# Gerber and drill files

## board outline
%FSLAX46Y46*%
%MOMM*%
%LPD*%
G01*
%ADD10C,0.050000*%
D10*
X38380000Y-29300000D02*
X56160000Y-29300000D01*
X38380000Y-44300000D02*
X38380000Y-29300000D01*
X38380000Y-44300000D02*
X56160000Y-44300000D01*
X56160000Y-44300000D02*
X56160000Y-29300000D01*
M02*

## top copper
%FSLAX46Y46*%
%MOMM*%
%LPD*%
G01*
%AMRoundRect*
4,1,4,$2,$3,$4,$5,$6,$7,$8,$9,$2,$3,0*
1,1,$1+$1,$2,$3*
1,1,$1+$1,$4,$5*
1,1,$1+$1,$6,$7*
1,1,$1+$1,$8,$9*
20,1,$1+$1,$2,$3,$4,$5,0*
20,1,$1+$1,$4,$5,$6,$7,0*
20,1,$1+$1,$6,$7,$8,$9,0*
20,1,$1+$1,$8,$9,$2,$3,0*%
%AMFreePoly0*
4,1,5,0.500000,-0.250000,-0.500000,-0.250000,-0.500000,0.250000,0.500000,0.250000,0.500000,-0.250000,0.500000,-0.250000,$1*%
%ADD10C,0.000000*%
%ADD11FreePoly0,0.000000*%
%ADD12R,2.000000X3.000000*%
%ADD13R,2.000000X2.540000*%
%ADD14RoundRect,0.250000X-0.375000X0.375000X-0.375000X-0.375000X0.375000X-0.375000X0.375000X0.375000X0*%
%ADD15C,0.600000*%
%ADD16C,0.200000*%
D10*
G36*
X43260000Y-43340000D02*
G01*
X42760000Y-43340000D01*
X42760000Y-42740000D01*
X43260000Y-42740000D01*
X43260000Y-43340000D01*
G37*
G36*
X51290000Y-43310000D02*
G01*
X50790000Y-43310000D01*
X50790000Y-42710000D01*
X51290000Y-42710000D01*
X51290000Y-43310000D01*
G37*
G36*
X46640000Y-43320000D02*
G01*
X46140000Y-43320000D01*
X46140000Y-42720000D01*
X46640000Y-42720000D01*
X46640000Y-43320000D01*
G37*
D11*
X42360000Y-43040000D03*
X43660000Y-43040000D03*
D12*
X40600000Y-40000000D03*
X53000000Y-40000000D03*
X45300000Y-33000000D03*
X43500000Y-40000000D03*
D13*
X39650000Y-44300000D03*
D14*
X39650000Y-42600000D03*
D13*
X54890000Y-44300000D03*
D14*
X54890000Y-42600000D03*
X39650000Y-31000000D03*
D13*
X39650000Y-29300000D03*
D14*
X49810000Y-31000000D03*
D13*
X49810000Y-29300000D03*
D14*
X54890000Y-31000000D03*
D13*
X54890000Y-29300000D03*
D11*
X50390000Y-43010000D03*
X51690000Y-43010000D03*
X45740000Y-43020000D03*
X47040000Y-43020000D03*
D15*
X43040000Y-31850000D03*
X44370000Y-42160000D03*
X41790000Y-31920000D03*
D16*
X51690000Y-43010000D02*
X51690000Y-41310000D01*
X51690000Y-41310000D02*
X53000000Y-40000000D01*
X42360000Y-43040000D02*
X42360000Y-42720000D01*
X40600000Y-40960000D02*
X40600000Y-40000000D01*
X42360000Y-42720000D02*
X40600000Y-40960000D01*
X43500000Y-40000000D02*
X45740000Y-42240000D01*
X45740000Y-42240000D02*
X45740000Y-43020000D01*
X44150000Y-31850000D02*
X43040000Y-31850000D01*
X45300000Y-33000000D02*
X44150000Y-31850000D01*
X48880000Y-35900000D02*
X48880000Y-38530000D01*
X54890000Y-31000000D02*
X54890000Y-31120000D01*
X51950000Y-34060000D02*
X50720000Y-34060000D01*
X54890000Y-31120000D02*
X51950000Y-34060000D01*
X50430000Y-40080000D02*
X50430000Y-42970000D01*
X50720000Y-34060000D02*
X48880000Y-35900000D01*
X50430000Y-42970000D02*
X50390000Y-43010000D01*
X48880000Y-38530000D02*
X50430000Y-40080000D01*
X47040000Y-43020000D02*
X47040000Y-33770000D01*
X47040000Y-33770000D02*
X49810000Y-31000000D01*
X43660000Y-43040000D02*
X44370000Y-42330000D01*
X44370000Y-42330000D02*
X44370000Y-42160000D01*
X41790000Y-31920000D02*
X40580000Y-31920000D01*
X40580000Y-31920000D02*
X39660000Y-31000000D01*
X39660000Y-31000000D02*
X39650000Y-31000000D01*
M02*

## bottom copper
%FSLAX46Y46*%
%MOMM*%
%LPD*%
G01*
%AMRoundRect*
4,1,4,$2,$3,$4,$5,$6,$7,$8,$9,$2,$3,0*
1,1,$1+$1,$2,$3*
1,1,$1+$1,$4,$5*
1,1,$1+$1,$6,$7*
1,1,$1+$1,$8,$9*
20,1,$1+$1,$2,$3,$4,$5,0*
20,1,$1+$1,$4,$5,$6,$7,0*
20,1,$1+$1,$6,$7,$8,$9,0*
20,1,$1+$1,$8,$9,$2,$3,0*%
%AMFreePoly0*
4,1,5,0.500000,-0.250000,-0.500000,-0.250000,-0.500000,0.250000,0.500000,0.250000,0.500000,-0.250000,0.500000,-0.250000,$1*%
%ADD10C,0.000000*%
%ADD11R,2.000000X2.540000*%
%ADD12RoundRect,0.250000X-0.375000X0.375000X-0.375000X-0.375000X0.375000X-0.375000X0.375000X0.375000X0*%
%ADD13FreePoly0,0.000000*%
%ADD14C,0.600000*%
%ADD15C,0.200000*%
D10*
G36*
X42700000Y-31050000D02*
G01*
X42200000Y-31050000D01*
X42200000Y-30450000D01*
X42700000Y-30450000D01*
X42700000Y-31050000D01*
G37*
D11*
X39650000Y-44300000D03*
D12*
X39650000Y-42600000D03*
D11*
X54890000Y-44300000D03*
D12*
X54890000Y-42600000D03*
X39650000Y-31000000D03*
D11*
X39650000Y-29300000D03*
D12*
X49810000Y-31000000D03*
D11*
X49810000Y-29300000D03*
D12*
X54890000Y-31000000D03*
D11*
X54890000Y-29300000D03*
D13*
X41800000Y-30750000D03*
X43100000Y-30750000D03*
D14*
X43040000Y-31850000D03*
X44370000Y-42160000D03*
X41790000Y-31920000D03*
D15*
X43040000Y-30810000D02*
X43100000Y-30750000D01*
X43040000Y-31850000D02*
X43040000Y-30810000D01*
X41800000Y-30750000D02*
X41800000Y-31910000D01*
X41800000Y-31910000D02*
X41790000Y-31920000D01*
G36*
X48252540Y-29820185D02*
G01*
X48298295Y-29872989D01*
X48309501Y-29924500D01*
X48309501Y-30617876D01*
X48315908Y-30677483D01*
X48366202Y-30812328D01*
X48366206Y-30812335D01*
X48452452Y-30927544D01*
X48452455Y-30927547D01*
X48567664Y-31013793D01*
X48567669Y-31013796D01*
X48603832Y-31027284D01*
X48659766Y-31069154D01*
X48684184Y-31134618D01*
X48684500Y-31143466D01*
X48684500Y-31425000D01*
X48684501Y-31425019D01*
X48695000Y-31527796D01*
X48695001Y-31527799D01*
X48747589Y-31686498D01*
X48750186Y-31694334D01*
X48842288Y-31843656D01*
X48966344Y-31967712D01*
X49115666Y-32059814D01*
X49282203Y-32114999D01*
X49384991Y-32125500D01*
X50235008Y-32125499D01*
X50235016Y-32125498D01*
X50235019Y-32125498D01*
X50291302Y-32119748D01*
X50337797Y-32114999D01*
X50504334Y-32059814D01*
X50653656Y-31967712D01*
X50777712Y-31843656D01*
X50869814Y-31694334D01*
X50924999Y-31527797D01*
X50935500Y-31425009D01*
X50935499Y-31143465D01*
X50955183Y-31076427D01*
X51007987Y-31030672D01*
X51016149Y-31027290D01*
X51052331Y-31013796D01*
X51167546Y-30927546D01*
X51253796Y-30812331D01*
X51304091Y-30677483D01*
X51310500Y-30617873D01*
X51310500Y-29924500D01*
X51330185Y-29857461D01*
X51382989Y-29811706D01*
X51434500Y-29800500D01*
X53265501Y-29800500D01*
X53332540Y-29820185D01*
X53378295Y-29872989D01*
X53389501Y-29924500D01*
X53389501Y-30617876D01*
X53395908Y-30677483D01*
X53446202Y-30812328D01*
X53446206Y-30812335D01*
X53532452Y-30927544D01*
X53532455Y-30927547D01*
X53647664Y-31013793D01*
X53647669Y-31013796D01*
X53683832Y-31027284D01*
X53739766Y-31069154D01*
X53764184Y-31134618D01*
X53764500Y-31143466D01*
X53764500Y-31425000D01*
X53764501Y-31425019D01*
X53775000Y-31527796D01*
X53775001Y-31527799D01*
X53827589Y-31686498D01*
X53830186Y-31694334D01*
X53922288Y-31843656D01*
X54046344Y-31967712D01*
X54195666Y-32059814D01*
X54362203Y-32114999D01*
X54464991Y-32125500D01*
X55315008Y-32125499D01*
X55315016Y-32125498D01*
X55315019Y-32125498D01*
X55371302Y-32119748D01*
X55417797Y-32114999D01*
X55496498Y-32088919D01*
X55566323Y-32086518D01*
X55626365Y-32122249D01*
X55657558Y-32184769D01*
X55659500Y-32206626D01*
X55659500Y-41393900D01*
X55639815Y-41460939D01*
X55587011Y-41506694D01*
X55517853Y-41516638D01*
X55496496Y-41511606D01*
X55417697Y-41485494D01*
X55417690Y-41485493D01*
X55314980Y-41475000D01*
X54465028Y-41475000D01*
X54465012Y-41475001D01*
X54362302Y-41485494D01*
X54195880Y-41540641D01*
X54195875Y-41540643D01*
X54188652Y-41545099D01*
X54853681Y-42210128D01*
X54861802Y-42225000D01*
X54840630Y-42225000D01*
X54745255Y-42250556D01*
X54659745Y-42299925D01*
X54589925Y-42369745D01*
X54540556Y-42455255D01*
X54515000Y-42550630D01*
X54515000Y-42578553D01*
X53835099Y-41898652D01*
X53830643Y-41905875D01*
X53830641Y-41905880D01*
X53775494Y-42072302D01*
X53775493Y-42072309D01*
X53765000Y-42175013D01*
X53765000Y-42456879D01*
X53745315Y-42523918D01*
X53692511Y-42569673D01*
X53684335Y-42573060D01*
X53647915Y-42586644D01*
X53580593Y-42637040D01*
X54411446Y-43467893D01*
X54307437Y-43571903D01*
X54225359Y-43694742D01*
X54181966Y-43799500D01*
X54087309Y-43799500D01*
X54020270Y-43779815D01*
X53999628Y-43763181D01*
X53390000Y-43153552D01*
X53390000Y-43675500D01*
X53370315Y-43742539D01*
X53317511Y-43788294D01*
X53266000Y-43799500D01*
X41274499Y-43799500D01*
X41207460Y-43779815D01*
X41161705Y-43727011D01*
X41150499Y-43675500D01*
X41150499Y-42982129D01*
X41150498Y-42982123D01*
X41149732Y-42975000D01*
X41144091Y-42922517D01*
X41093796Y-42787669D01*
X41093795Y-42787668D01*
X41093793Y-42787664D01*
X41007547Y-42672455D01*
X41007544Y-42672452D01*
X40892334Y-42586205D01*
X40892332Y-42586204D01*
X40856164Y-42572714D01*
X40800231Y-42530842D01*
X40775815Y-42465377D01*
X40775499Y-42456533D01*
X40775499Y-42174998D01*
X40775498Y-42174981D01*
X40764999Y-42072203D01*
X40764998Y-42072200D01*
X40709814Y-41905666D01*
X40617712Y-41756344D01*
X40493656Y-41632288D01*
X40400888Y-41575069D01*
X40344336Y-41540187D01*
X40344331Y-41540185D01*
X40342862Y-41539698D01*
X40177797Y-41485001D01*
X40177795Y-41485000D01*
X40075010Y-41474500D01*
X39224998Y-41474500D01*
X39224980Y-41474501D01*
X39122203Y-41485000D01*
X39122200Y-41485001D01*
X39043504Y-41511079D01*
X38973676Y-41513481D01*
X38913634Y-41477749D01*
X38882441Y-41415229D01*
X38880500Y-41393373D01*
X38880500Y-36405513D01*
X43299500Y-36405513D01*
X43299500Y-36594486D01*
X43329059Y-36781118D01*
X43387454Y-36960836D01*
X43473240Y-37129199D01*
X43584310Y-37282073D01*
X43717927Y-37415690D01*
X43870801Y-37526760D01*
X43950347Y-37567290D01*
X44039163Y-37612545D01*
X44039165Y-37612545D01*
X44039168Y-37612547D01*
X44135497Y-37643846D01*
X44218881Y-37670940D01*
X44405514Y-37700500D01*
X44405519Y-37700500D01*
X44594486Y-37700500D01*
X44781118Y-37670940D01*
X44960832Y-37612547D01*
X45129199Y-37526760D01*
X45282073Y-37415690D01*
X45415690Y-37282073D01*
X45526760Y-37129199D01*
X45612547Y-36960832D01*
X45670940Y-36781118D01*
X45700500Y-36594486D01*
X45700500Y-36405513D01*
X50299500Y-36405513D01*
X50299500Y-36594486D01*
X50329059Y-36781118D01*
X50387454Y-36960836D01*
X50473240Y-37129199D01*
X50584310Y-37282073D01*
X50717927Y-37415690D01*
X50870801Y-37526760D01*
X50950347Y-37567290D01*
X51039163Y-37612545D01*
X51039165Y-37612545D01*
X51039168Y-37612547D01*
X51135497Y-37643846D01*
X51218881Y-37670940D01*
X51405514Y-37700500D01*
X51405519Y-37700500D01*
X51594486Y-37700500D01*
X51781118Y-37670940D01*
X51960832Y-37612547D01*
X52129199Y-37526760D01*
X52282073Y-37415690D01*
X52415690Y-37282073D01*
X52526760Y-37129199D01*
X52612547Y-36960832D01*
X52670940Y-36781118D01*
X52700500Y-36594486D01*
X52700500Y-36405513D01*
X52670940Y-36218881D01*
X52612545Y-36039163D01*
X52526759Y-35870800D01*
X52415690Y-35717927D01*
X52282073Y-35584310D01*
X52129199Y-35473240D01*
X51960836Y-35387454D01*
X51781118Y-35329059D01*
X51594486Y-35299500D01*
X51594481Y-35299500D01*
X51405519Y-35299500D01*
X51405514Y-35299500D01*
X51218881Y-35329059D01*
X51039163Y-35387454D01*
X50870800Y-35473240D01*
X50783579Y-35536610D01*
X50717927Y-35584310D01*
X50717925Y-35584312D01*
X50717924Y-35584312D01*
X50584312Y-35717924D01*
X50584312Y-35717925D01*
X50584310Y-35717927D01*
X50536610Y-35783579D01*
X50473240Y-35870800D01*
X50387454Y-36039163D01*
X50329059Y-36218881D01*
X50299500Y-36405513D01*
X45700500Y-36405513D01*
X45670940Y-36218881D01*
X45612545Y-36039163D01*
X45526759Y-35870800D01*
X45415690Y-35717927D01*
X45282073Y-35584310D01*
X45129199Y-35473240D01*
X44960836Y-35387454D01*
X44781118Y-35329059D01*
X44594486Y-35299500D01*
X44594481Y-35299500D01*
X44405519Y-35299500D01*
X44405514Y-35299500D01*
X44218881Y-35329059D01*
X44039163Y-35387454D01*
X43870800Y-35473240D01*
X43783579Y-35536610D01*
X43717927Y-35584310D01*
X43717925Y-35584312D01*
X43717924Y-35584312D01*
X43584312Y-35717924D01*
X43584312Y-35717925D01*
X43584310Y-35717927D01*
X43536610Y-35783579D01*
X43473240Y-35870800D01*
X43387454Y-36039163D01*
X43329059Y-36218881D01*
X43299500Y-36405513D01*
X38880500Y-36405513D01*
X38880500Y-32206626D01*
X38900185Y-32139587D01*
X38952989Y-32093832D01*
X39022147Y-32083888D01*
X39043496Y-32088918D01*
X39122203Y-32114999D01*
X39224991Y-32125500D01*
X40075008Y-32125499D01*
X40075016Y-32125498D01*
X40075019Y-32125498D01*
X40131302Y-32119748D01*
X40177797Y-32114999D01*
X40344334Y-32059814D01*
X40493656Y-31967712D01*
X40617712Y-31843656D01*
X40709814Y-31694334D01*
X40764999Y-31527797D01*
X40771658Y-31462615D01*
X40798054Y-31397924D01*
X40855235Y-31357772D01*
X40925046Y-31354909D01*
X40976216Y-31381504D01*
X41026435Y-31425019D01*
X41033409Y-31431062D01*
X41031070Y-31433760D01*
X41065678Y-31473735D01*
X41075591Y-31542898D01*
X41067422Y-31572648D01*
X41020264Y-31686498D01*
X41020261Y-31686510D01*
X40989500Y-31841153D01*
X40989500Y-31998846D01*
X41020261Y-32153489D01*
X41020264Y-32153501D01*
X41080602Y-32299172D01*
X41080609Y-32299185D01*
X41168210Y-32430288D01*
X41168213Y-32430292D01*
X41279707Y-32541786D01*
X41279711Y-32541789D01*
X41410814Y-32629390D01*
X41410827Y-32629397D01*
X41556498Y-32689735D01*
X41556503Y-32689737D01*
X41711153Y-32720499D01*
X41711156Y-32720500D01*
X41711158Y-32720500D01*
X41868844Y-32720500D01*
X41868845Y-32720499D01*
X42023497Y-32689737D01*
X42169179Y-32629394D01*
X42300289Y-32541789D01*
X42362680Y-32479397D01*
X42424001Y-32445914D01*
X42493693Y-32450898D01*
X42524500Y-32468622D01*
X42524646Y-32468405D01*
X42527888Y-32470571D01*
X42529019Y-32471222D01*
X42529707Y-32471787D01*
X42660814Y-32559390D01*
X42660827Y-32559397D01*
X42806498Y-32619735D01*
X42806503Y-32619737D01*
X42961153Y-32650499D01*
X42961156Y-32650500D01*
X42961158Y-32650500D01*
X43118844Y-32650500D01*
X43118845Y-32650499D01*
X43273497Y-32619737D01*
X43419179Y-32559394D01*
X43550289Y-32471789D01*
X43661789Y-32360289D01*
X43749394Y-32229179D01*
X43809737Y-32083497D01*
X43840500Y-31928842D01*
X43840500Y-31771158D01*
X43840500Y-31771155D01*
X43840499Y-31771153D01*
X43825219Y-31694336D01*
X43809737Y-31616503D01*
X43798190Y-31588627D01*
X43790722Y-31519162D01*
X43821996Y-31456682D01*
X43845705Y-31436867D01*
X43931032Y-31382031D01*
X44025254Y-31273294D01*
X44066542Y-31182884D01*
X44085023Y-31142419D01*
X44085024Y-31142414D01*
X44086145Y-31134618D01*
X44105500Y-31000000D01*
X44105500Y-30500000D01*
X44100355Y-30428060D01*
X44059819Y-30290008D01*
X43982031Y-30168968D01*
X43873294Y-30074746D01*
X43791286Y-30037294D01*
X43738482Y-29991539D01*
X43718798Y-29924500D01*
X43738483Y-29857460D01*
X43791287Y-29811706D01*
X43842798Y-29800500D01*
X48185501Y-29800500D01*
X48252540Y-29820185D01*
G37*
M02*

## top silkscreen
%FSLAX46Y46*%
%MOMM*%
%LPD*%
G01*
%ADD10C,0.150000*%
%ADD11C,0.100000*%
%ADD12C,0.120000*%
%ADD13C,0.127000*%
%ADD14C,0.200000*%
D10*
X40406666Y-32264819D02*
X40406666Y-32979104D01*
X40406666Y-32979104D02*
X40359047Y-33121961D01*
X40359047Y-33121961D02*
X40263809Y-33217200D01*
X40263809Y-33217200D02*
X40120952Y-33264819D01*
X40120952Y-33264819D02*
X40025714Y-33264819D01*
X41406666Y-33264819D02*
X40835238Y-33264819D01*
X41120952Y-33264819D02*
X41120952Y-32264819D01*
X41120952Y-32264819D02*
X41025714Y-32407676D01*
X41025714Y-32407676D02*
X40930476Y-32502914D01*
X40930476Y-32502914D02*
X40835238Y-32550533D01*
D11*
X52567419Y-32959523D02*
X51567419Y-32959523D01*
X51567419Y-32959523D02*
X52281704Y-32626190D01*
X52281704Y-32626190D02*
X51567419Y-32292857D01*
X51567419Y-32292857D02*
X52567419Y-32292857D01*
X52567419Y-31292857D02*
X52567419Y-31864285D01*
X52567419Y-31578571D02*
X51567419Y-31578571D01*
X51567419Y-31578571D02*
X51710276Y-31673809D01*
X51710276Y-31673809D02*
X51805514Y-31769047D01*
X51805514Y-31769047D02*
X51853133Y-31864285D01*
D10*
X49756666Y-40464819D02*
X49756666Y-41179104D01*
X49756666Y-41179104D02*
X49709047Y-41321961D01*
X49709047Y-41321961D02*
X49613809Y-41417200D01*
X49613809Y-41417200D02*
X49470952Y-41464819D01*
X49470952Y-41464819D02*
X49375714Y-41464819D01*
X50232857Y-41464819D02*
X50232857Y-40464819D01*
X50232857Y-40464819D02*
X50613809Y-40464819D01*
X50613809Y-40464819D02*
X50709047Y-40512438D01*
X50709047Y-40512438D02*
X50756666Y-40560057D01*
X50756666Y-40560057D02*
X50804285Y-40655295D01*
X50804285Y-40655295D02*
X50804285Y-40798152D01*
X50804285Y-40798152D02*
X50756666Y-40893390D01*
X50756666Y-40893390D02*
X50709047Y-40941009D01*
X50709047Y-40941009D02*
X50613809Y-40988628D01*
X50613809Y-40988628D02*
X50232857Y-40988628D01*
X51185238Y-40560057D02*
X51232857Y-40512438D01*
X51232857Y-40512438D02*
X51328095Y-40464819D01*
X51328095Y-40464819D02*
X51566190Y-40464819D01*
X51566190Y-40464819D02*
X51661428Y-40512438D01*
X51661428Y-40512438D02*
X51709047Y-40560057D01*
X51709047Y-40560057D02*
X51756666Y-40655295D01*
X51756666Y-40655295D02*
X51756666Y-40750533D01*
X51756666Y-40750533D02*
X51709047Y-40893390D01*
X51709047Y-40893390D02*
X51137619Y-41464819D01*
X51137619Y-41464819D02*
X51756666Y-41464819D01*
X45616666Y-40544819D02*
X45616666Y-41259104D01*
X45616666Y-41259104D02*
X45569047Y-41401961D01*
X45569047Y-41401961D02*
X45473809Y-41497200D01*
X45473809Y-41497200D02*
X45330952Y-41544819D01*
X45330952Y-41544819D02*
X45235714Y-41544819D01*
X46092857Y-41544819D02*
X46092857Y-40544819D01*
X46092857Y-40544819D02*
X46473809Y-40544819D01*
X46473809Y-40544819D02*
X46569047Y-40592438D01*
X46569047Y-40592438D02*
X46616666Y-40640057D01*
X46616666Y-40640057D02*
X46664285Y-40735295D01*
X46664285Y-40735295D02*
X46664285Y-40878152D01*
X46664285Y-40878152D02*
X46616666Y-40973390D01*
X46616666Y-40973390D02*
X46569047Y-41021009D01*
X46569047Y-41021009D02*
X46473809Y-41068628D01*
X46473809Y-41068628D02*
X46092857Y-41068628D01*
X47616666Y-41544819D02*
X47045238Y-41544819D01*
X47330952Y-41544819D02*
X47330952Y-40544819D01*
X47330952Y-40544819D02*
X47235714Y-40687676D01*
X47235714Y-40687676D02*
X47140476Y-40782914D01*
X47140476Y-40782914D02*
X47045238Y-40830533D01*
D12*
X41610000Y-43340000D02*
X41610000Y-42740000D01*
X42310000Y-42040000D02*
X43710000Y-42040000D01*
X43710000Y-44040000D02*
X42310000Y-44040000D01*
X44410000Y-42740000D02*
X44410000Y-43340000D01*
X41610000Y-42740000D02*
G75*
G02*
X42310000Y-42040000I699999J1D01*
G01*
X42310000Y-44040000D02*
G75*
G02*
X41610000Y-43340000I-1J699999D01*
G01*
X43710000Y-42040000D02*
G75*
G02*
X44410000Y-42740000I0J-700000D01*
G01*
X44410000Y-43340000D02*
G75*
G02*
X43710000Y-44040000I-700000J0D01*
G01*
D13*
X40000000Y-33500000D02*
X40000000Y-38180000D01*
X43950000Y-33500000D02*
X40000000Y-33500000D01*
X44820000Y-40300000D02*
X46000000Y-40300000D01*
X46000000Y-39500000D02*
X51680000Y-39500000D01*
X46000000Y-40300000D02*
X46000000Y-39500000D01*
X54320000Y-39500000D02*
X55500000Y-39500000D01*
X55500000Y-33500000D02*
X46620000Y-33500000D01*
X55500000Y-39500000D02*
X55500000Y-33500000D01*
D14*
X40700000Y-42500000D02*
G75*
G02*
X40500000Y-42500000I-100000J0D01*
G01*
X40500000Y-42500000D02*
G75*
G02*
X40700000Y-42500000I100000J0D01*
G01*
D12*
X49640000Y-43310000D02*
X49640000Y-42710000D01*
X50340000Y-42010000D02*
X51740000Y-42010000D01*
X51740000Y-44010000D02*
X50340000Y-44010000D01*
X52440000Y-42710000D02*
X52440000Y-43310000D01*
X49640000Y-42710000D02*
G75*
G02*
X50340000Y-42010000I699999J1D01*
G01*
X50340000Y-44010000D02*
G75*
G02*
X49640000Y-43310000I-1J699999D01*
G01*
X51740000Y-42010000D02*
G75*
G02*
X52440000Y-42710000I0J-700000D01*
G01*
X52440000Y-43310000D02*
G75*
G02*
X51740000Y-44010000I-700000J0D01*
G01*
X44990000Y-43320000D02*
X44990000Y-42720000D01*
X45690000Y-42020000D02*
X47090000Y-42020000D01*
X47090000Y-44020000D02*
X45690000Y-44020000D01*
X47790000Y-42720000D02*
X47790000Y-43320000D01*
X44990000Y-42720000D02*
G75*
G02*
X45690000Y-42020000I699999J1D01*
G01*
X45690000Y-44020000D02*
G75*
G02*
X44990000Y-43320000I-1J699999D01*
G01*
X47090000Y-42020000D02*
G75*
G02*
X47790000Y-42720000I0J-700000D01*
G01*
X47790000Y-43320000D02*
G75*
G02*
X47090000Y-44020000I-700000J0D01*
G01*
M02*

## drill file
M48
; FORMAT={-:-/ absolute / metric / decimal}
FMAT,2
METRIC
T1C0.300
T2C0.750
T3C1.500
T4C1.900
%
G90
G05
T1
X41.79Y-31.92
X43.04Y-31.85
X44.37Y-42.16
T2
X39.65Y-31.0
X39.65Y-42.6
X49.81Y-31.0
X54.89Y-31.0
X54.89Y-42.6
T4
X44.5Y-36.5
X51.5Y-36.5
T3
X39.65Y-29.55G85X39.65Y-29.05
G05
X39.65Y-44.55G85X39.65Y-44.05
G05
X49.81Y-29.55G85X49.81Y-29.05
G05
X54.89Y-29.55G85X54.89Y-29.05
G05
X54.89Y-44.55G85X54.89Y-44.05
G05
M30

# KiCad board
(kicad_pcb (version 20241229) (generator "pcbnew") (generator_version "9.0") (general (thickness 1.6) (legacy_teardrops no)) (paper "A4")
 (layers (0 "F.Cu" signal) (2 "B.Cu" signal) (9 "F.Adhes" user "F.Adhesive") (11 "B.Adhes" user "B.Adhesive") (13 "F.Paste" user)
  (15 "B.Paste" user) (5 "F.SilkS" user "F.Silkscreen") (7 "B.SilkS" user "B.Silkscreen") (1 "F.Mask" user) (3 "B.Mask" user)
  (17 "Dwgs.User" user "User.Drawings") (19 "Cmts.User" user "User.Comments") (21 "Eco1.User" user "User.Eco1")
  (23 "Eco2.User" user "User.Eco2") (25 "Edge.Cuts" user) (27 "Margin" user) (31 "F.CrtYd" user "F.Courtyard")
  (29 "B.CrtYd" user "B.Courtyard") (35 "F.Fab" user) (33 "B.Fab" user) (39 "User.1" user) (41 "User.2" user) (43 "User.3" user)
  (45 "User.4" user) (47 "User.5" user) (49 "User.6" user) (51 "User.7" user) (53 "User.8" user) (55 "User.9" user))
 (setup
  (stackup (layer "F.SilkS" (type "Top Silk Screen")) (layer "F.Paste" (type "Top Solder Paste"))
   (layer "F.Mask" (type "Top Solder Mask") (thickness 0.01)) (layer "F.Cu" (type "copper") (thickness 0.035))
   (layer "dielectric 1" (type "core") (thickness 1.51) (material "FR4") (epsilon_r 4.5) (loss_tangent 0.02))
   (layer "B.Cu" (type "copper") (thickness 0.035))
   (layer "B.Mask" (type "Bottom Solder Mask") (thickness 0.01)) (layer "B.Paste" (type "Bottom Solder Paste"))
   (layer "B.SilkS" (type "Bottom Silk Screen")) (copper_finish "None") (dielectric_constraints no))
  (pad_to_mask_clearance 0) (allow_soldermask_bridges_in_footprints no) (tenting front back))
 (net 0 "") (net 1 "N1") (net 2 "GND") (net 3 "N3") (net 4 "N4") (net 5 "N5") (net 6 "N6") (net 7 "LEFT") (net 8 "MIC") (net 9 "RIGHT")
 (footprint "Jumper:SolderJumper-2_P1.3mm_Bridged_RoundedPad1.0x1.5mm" (layer "F.Cu") (at 43.01 43.04)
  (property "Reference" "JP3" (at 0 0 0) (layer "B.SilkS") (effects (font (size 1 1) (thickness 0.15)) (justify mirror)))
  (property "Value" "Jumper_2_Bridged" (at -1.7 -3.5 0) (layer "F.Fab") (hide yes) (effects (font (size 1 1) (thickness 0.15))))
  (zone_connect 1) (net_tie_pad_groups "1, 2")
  (fp_poly (pts (xy 0.25 -0.3) (xy -0.25 -0.3) (xy -0.25 0.3) (xy 0.25 0.3)) (stroke (width 0) (type solid)) (fill yes) (layer "F.Cu"))
  (fp_line (start -1.4 0.3) (end -1.4 -0.3) (stroke (width 0.12) (type solid)) (layer "F.SilkS"))
  (fp_line (start -0.7 -1) (end 0.7 -1) (stroke (width 0.12) (type solid)) (layer "F.SilkS"))
  (fp_line (start 0.7 1) (end -0.7 1) (stroke (width 0.12) (type solid)) (layer "F.SilkS"))
  (fp_line (start 1.4 -0.3) (end 1.4 0.3) (stroke (width 0.12) (type solid)) (layer "F.SilkS"))
  (fp_arc (start -1.4 -0.3) (mid -1.194975 -0.794975) (end -0.7 -1) (stroke (width 0.12) (type solid)) (layer "F.SilkS"))
  (fp_arc (start -0.7 1) (mid -1.194975 0.794975) (end -1.4 0.3) (stroke (width 0.12) (type solid)) (layer "F.SilkS"))
  (fp_arc (start 0.7 -1) (mid 1.194975 -0.794975) (end 1.4 -0.3) (stroke (width 0.12) (type solid)) (layer "F.SilkS"))
  (fp_arc (start 1.4 0.3) (mid 1.194975 0.794975) (end 0.7 1) (stroke (width 0.12) (type solid)) (layer "F.SilkS"))
  (pad "1" smd custom (at -0.65 0) (size 1 0.5) (layers "F.Cu" "F.Mask") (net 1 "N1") (zone_connect 2) (thermal_bridge_angle 45)
   (options (clearance outline) (anchor rect)) (primitives))
  (pad "2" smd custom (at 0.65 0) (size 1 0.5) (layers "F.Cu" "F.Mask") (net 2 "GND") (zone_connect 2) (thermal_bridge_angle 45)
   (options (clearance outline) (anchor rect)) (primitives)))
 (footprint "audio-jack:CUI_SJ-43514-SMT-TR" (layer "F.Cu") (at 40.6 40)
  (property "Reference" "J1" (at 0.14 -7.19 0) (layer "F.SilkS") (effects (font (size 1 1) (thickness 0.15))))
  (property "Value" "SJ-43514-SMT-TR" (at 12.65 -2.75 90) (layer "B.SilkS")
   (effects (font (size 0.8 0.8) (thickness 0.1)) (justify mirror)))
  (fp_line (start -0.6 -6.5) (end -0.6 -1.82) (stroke (width 0.127) (type solid)) (layer "F.SilkS"))
  (fp_line (start 3.35 -6.5) (end -0.6 -6.5) (stroke (width 0.127) (type solid)) (layer "F.SilkS"))
  (fp_line (start 4.22 0.3) (end 5.4 0.3) (stroke (width 0.127) (type solid)) (layer "F.SilkS"))
  (fp_line (start 5.4 -0.5) (end 11.08 -0.5) (stroke (width 0.127) (type solid)) (layer "F.SilkS"))
  (fp_line (start 5.4 0.3) (end 5.4 -0.5) (stroke (width 0.127) (type solid)) (layer "F.SilkS"))
  (fp_line (start 13.72 -0.5) (end 14.9 -0.5) (stroke (width 0.127) (type solid)) (layer "F.SilkS"))
  (fp_line (start 14.9 -6.5) (end 6.02 -6.5) (stroke (width 0.127) (type solid)) (layer "F.SilkS"))
  (fp_line (start 14.9 -0.5) (end 14.9 -6.5) (stroke (width 0.127) (type solid)) (layer "F.SilkS"))
  (fp_circle (center 0 2.5) (end 0.1 2.5) (stroke (width 0.2) (type solid)) (fill no) (layer "F.SilkS"))
  (pad "" np_thru_hole circle (at 3.9 -3.5) (size 1.9 1.9) (drill 1.9) (layers "*.Cu" "*.Mask"))
  (pad "" np_thru_hole circle (at 10.9 -3.5) (size 1.9 1.9) (drill 1.9) (layers "*.Cu" "*.Mask"))
  (pad "1" smd rect (at 0 0) (size 2 3) (layers "F.Cu" "F.Mask" "F.Paste") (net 1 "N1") (solder_mask_margin 0.102))
  (pad "2" smd rect (at 12.4 0) (size 2 3) (layers "F.Cu" "F.Mask" "F.Paste") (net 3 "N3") (solder_mask_margin 0.102))
  (pad "3" smd rect (at 4.7 -7) (size 2 3) (layers "F.Cu" "F.Mask" "F.Paste") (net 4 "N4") (solder_mask_margin 0.102))
  (pad "4" smd rect (at 2.9 0) (size 2 3) (layers "F.Cu" "F.Mask" "F.Paste") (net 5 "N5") (solder_mask_margin 0.102)))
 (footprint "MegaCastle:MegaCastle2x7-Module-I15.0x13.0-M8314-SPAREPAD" (layer "F.Cu") (at 47.27 36.8 90)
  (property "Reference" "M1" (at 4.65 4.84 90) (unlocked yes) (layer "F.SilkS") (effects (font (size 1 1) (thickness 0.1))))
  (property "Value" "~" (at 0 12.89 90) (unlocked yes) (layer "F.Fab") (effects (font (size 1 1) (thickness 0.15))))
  (fp_line (start 7.5 -8.89) (end 7.5 8.89) (stroke (width 0.05) (type default)) (layer "Edge.Cuts"))
  (fp_line (start -7.5 -8.89) (end 7.5 -8.89) (stroke (width 0.05) (type default)) (layer "Edge.Cuts"))
  (fp_line (start -7.5 -8.89) (end -7.5 8.89) (stroke (width 0.05) (type default)) (layer "Edge.Cuts"))
  (fp_line (start -7.5 8.89) (end 7.5 8.89) (stroke (width 0.05) (type default)) (layer "Edge.Cuts"))
  (pad "1" thru_hole rect (at -7.5 -7.62 90) (size 2.54 2) (drill oval 2 1.5) (layers "*.Cu" "*.Mask") (remove_unused_layers no)
   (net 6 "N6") (thermal_bridge_angle 45))
  (pad "1" thru_hole roundrect (at -5.8 -7.62 270) (size 1.25 1.25) (drill 0.75) (layers "*.Cu" "*.Mask") (remove_unused_layers no)
   (roundrect_rratio 0.2) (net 6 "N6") (thermal_bridge_angle 45))
  (pad "7" thru_hole rect (at -7.5 7.62 90) (size 2.54 2) (drill oval 2 1.5) (layers "*.Cu" "*.Mask") (remove_unused_layers no)
   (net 2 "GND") (thermal_bridge_angle 45))
  (pad "7" thru_hole roundrect (at -5.8 7.62 270) (size 1.25 1.25) (drill 0.75) (layers "*.Cu" "*.Mask") (remove_unused_layers no)
   (roundrect_rratio 0.2) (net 2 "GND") (thermal_bridge_angle 45))
  (pad "8" thru_hole roundrect (at 5.8 -7.62 270) (size 1.25 1.25) (drill 0.75) (layers "*.Cu" "*.Mask") (remove_unused_layers no)
   (roundrect_rratio 0.2) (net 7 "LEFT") (thermal_bridge_angle 45))
  (pad "8" thru_hole rect (at 7.5 -7.62 90) (size 2.54 2) (drill oval 2 1.5) (layers "*.Cu" "*.Mask") (remove_unused_layers no)
   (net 7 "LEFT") (thermal_bridge_angle 45))
  (pad "12" thru_hole roundrect (at 5.8 2.54 270) (size 1.25 1.25) (drill 0.75) (layers "*.Cu" "*.Mask") (remove_unused_layers no)
   (roundrect_rratio 0.2) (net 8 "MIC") (thermal_bridge_angle 45))
  (pad "12" thru_hole rect (at 7.5 2.54 90) (size 2.54 2) (drill oval 2 1.5) (layers "*.Cu" "*.Mask") (remove_unused_layers no)
   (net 8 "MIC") (thermal_bridge_angle 45))
  (pad "14" thru_hole roundrect (at 5.8 7.62 270) (size 1.25 1.25) (drill 0.75) (layers "*.Cu" "*.Mask") (remove_unused_layers no)
   (roundrect_rratio 0.2) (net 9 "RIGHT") (thermal_bridge_angle 45))
  (pad "14" thru_hole rect (at 7.5 7.62 90) (size 2.54 2) (drill oval 2 1.5) (layers "*.Cu" "*.Mask") (remove_unused_layers no)
   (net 9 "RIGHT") (thermal_bridge_angle 45))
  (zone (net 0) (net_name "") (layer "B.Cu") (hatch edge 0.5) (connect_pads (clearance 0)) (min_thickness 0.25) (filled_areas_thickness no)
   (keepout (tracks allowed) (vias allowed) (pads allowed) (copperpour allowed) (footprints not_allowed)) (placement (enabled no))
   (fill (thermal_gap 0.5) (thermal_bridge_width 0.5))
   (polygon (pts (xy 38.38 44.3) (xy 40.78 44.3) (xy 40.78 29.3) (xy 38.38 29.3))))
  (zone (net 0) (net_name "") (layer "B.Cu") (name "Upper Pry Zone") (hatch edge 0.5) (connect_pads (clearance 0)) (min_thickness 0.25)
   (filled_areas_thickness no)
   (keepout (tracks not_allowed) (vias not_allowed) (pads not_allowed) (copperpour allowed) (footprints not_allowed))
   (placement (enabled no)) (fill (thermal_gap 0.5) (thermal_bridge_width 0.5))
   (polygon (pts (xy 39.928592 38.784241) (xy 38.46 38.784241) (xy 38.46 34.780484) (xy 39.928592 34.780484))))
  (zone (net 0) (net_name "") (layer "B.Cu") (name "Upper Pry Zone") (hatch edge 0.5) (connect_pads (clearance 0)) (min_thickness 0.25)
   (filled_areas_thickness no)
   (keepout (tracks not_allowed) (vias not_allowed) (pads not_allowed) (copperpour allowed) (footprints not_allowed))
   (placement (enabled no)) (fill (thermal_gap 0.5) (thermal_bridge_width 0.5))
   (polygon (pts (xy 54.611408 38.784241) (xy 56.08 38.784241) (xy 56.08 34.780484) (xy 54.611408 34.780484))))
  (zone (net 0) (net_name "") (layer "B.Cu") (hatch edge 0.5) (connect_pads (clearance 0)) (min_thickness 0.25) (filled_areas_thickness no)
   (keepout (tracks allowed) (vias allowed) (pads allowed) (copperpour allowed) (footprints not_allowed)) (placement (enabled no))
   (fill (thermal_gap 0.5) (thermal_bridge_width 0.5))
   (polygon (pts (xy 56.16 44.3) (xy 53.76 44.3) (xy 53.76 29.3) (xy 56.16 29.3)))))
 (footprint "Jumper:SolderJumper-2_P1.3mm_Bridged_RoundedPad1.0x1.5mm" (layer "F.Cu") (at 51.04 43.01)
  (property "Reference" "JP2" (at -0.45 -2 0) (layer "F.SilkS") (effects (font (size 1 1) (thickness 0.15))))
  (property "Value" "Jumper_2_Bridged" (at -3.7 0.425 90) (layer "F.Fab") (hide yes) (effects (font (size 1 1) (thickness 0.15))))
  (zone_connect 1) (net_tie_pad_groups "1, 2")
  (fp_poly (pts (xy 0.25 -0.3) (xy -0.25 -0.3) (xy -0.25 0.3) (xy 0.25 0.3)) (stroke (width 0) (type solid)) (fill yes) (layer "F.Cu"))
  (fp_line (start -1.4 0.3) (end -1.4 -0.3) (stroke (width 0.12) (type solid)) (layer "F.SilkS"))
  (fp_line (start -0.7 -1) (end 0.7 -1) (stroke (width 0.12) (type solid)) (layer "F.SilkS"))
  (fp_line (start 0.7 1) (end -0.7 1) (stroke (width 0.12) (type solid)) (layer "F.SilkS"))
  (fp_line (start 1.4 -0.3) (end 1.4 0.3) (stroke (width 0.12) (type solid)) (layer "F.SilkS"))
  (fp_arc (start -1.4 -0.3) (mid -1.194975 -0.794975) (end -0.7 -1) (stroke (width 0.12) (type solid)) (layer "F.SilkS"))
  (fp_arc (start -0.7 1) (mid -1.194975 0.794975) (end -1.4 0.3) (stroke (width 0.12) (type solid)) (layer "F.SilkS"))
  (fp_arc (start 0.7 -1) (mid 1.194975 -0.794975) (end 1.4 -0.3) (stroke (width 0.12) (type solid)) (layer "F.SilkS"))
  (fp_arc (start 1.4 0.3) (mid 1.194975 0.794975) (end 0.7 1) (stroke (width 0.12) (type solid)) (layer "F.SilkS"))
  (pad "1" smd custom (at -0.65 0) (size 1 0.5) (layers "F.Cu" "F.Mask") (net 9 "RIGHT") (zone_connect 2) (thermal_bridge_angle 45)
   (options (clearance outline) (anchor rect)) (primitives))
  (pad "2" smd custom (at 0.65 0) (size 1 0.5) (layers "F.Cu" "F.Mask") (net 3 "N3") (zone_connect 2) (thermal_bridge_angle 45)
   (options (clearance outline) (anchor rect)) (primitives)))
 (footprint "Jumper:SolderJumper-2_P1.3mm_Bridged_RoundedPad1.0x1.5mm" (layer "F.Cu") (at 46.39 43.02)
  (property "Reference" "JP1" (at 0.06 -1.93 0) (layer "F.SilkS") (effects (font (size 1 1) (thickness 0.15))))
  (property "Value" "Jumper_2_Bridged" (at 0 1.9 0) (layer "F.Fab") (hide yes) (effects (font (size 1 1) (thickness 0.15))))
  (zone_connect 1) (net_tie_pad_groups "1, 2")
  (fp_poly (pts (xy 0.25 -0.3) (xy -0.25 -0.3) (xy -0.25 0.3) (xy 0.25 0.3)) (stroke (width 0) (type solid)) (fill yes) (layer "F.Cu"))
  (fp_line (start -1.4 0.3) (end -1.4 -0.3) (stroke (width 0.12) (type solid)) (layer "F.SilkS"))
  (fp_line (start -0.7 -1) (end 0.7 -1) (stroke (width 0.12) (type solid)) (layer "F.SilkS"))
  (fp_line (start 0.7 1) (end -0.7 1) (stroke (width 0.12) (type solid)) (layer "F.SilkS"))
  (fp_line (start 1.4 -0.3) (end 1.4 0.3) (stroke (width 0.12) (type solid)) (layer "F.SilkS"))
  (fp_arc (start -1.4 -0.3) (mid -1.194975 -0.794975) (end -0.7 -1) (stroke (width 0.12) (type solid)) (layer "F.SilkS"))
  (fp_arc (start -0.7 1) (mid -1.194975 0.794975) (end -1.4 0.3) (stroke (width 0.12) (type solid)) (layer "F.SilkS"))
  (fp_arc (start 0.7 -1) (mid 1.194975 -0.794975) (end 1.4 -0.3) (stroke (width 0.12) (type solid)) (layer "F.SilkS"))
  (fp_arc (start 1.4 0.3) (mid 1.194975 0.794975) (end 0.7 1) (stroke (width 0.12) (type solid)) (layer "F.SilkS"))
  (pad "1" smd custom (at -0.65 0) (size 1 0.5) (layers "F.Cu" "F.Mask") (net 5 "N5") (zone_connect 2) (thermal_bridge_angle 45)
   (options (clearance outline) (anchor rect)) (primitives))
  (pad "2" smd custom (at 0.65 0) (size 1 0.5) (layers "F.Cu" "F.Mask") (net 8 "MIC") (zone_connect 2) (thermal_bridge_angle 45)
   (options (clearance outline) (anchor rect)) (primitives)))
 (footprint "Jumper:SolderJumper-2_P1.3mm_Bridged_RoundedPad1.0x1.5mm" (layer "B.Cu") (at 42.45 30.75)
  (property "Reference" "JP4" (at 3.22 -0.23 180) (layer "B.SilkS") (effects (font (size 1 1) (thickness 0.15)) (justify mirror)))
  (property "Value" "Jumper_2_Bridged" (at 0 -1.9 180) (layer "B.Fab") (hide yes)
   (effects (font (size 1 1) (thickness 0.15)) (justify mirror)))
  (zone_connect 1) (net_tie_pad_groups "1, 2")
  (fp_poly (pts (xy 0.25 0.3) (xy -0.25 0.3) (xy -0.25 -0.3) (xy 0.25 -0.3)) (stroke (width 0) (type solid)) (fill yes) (layer "B.Cu"))
  (pad "1" smd custom (at -0.65 0) (size 1 0.5) (layers "B.Cu" "B.Mask") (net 7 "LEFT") (zone_connect 2) (thermal_bridge_angle 45)
   (options (clearance outline) (anchor rect)) (primitives))
  (pad "2" smd custom (at 0.65 0) (size 1 0.5) (layers "B.Cu" "B.Mask") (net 4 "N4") (zone_connect 2) (thermal_bridge_angle 45)
   (options (clearance outline) (anchor rect)) (primitives)))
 (segment (start 51.69 43.01) (end 51.69 41.31) (width 0.2) (layer "F.Cu") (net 3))
 (segment (start 51.69 41.31) (end 53 40) (width 0.2) (layer "F.Cu") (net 3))
 (segment (start 42.36 43.04) (end 42.36 42.72) (width 0.2) (layer "F.Cu") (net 1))
 (segment (start 40.6 40.96) (end 40.6 40) (width 0.2) (layer "F.Cu") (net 1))
 (segment (start 42.36 42.72) (end 40.6 40.96) (width 0.2) (layer "F.Cu") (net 1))
 (segment (start 43.5 40) (end 45.74 42.24) (width 0.2) (layer "F.Cu") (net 5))
 (segment (start 45.74 42.24) (end 45.74 43.02) (width 0.2) (layer "F.Cu") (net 5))
 (segment (start 44.15 31.85) (end 43.04 31.85) (width 0.2) (layer "F.Cu") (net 4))
 (segment (start 45.3 33) (end 44.15 31.85) (width 0.2) (layer "F.Cu") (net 4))
 (via (at 43.04 31.85) (size 0.6) (drill 0.3) (layers "F.Cu" "B.Cu") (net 4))
 (segment (start 43.04 30.81) (end 43.1 30.75) (width 0.2) (layer "B.Cu") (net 4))
 (segment (start 43.04 31.85) (end 43.04 30.81) (width 0.2) (layer "B.Cu") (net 4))
 (segment (start 48.88 35.9) (end 48.88 38.53) (width 0.2) (layer "F.Cu") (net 9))
 (segment (start 54.89 31) (end 54.89 31.12) (width 0.2) (layer "F.Cu") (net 9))
 (segment (start 51.95 34.06) (end 50.72 34.06) (width 0.2) (layer "F.Cu") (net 9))
 (segment (start 54.89 31.12) (end 51.95 34.06) (width 0.2) (layer "F.Cu") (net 9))
 (segment (start 50.43 40.08) (end 50.43 42.97) (width 0.2) (layer "F.Cu") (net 9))
 (segment (start 50.72 34.06) (end 48.88 35.9) (width 0.2) (layer "F.Cu") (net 9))
 (segment (start 50.43 42.97) (end 50.39 43.01) (width 0.2) (layer "F.Cu") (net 9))
 (segment (start 48.88 38.53) (end 50.43 40.08) (width 0.2) (layer "F.Cu") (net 9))
 (segment (start 47.04 43.02) (end 47.04 33.77) (width 0.2) (layer "F.Cu") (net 8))
 (segment (start 47.04 33.77) (end 49.81 31) (width 0.2) (layer "F.Cu") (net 8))
 (segment (start 43.66 43.04) (end 44.37 42.33) (width 0.2) (layer "F.Cu") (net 2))
 (segment (start 44.37 42.33) (end 44.37 42.16) (width 0.2) (layer "F.Cu") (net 2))
 (via (at 44.37 42.16) (size 0.6) (drill 0.3) (layers "F.Cu" "B.Cu") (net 2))
 (segment (start 41.79 31.92) (end 40.58 31.92) (width 0.2) (layer "F.Cu") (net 7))
 (segment (start 40.58 31.92) (end 39.66 31) (width 0.2) (layer "F.Cu") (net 7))
 (segment (start 39.66 31) (end 39.65 31) (width 0.2) (layer "F.Cu") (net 7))
 (via (at 41.79 31.92) (size 0.6) (drill 0.3) (layers "F.Cu" "B.Cu") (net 7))
 (segment (start 41.8 30.75) (end 41.8 31.91) (width 0.2) (layer "B.Cu") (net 7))
 (segment (start 41.8 31.91) (end 41.79 31.92) (width 0.2) (layer "B.Cu") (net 7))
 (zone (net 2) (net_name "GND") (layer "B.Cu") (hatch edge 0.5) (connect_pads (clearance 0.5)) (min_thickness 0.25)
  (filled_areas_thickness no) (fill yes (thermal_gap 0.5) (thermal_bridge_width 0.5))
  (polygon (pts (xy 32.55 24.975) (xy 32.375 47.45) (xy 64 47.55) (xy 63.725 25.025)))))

